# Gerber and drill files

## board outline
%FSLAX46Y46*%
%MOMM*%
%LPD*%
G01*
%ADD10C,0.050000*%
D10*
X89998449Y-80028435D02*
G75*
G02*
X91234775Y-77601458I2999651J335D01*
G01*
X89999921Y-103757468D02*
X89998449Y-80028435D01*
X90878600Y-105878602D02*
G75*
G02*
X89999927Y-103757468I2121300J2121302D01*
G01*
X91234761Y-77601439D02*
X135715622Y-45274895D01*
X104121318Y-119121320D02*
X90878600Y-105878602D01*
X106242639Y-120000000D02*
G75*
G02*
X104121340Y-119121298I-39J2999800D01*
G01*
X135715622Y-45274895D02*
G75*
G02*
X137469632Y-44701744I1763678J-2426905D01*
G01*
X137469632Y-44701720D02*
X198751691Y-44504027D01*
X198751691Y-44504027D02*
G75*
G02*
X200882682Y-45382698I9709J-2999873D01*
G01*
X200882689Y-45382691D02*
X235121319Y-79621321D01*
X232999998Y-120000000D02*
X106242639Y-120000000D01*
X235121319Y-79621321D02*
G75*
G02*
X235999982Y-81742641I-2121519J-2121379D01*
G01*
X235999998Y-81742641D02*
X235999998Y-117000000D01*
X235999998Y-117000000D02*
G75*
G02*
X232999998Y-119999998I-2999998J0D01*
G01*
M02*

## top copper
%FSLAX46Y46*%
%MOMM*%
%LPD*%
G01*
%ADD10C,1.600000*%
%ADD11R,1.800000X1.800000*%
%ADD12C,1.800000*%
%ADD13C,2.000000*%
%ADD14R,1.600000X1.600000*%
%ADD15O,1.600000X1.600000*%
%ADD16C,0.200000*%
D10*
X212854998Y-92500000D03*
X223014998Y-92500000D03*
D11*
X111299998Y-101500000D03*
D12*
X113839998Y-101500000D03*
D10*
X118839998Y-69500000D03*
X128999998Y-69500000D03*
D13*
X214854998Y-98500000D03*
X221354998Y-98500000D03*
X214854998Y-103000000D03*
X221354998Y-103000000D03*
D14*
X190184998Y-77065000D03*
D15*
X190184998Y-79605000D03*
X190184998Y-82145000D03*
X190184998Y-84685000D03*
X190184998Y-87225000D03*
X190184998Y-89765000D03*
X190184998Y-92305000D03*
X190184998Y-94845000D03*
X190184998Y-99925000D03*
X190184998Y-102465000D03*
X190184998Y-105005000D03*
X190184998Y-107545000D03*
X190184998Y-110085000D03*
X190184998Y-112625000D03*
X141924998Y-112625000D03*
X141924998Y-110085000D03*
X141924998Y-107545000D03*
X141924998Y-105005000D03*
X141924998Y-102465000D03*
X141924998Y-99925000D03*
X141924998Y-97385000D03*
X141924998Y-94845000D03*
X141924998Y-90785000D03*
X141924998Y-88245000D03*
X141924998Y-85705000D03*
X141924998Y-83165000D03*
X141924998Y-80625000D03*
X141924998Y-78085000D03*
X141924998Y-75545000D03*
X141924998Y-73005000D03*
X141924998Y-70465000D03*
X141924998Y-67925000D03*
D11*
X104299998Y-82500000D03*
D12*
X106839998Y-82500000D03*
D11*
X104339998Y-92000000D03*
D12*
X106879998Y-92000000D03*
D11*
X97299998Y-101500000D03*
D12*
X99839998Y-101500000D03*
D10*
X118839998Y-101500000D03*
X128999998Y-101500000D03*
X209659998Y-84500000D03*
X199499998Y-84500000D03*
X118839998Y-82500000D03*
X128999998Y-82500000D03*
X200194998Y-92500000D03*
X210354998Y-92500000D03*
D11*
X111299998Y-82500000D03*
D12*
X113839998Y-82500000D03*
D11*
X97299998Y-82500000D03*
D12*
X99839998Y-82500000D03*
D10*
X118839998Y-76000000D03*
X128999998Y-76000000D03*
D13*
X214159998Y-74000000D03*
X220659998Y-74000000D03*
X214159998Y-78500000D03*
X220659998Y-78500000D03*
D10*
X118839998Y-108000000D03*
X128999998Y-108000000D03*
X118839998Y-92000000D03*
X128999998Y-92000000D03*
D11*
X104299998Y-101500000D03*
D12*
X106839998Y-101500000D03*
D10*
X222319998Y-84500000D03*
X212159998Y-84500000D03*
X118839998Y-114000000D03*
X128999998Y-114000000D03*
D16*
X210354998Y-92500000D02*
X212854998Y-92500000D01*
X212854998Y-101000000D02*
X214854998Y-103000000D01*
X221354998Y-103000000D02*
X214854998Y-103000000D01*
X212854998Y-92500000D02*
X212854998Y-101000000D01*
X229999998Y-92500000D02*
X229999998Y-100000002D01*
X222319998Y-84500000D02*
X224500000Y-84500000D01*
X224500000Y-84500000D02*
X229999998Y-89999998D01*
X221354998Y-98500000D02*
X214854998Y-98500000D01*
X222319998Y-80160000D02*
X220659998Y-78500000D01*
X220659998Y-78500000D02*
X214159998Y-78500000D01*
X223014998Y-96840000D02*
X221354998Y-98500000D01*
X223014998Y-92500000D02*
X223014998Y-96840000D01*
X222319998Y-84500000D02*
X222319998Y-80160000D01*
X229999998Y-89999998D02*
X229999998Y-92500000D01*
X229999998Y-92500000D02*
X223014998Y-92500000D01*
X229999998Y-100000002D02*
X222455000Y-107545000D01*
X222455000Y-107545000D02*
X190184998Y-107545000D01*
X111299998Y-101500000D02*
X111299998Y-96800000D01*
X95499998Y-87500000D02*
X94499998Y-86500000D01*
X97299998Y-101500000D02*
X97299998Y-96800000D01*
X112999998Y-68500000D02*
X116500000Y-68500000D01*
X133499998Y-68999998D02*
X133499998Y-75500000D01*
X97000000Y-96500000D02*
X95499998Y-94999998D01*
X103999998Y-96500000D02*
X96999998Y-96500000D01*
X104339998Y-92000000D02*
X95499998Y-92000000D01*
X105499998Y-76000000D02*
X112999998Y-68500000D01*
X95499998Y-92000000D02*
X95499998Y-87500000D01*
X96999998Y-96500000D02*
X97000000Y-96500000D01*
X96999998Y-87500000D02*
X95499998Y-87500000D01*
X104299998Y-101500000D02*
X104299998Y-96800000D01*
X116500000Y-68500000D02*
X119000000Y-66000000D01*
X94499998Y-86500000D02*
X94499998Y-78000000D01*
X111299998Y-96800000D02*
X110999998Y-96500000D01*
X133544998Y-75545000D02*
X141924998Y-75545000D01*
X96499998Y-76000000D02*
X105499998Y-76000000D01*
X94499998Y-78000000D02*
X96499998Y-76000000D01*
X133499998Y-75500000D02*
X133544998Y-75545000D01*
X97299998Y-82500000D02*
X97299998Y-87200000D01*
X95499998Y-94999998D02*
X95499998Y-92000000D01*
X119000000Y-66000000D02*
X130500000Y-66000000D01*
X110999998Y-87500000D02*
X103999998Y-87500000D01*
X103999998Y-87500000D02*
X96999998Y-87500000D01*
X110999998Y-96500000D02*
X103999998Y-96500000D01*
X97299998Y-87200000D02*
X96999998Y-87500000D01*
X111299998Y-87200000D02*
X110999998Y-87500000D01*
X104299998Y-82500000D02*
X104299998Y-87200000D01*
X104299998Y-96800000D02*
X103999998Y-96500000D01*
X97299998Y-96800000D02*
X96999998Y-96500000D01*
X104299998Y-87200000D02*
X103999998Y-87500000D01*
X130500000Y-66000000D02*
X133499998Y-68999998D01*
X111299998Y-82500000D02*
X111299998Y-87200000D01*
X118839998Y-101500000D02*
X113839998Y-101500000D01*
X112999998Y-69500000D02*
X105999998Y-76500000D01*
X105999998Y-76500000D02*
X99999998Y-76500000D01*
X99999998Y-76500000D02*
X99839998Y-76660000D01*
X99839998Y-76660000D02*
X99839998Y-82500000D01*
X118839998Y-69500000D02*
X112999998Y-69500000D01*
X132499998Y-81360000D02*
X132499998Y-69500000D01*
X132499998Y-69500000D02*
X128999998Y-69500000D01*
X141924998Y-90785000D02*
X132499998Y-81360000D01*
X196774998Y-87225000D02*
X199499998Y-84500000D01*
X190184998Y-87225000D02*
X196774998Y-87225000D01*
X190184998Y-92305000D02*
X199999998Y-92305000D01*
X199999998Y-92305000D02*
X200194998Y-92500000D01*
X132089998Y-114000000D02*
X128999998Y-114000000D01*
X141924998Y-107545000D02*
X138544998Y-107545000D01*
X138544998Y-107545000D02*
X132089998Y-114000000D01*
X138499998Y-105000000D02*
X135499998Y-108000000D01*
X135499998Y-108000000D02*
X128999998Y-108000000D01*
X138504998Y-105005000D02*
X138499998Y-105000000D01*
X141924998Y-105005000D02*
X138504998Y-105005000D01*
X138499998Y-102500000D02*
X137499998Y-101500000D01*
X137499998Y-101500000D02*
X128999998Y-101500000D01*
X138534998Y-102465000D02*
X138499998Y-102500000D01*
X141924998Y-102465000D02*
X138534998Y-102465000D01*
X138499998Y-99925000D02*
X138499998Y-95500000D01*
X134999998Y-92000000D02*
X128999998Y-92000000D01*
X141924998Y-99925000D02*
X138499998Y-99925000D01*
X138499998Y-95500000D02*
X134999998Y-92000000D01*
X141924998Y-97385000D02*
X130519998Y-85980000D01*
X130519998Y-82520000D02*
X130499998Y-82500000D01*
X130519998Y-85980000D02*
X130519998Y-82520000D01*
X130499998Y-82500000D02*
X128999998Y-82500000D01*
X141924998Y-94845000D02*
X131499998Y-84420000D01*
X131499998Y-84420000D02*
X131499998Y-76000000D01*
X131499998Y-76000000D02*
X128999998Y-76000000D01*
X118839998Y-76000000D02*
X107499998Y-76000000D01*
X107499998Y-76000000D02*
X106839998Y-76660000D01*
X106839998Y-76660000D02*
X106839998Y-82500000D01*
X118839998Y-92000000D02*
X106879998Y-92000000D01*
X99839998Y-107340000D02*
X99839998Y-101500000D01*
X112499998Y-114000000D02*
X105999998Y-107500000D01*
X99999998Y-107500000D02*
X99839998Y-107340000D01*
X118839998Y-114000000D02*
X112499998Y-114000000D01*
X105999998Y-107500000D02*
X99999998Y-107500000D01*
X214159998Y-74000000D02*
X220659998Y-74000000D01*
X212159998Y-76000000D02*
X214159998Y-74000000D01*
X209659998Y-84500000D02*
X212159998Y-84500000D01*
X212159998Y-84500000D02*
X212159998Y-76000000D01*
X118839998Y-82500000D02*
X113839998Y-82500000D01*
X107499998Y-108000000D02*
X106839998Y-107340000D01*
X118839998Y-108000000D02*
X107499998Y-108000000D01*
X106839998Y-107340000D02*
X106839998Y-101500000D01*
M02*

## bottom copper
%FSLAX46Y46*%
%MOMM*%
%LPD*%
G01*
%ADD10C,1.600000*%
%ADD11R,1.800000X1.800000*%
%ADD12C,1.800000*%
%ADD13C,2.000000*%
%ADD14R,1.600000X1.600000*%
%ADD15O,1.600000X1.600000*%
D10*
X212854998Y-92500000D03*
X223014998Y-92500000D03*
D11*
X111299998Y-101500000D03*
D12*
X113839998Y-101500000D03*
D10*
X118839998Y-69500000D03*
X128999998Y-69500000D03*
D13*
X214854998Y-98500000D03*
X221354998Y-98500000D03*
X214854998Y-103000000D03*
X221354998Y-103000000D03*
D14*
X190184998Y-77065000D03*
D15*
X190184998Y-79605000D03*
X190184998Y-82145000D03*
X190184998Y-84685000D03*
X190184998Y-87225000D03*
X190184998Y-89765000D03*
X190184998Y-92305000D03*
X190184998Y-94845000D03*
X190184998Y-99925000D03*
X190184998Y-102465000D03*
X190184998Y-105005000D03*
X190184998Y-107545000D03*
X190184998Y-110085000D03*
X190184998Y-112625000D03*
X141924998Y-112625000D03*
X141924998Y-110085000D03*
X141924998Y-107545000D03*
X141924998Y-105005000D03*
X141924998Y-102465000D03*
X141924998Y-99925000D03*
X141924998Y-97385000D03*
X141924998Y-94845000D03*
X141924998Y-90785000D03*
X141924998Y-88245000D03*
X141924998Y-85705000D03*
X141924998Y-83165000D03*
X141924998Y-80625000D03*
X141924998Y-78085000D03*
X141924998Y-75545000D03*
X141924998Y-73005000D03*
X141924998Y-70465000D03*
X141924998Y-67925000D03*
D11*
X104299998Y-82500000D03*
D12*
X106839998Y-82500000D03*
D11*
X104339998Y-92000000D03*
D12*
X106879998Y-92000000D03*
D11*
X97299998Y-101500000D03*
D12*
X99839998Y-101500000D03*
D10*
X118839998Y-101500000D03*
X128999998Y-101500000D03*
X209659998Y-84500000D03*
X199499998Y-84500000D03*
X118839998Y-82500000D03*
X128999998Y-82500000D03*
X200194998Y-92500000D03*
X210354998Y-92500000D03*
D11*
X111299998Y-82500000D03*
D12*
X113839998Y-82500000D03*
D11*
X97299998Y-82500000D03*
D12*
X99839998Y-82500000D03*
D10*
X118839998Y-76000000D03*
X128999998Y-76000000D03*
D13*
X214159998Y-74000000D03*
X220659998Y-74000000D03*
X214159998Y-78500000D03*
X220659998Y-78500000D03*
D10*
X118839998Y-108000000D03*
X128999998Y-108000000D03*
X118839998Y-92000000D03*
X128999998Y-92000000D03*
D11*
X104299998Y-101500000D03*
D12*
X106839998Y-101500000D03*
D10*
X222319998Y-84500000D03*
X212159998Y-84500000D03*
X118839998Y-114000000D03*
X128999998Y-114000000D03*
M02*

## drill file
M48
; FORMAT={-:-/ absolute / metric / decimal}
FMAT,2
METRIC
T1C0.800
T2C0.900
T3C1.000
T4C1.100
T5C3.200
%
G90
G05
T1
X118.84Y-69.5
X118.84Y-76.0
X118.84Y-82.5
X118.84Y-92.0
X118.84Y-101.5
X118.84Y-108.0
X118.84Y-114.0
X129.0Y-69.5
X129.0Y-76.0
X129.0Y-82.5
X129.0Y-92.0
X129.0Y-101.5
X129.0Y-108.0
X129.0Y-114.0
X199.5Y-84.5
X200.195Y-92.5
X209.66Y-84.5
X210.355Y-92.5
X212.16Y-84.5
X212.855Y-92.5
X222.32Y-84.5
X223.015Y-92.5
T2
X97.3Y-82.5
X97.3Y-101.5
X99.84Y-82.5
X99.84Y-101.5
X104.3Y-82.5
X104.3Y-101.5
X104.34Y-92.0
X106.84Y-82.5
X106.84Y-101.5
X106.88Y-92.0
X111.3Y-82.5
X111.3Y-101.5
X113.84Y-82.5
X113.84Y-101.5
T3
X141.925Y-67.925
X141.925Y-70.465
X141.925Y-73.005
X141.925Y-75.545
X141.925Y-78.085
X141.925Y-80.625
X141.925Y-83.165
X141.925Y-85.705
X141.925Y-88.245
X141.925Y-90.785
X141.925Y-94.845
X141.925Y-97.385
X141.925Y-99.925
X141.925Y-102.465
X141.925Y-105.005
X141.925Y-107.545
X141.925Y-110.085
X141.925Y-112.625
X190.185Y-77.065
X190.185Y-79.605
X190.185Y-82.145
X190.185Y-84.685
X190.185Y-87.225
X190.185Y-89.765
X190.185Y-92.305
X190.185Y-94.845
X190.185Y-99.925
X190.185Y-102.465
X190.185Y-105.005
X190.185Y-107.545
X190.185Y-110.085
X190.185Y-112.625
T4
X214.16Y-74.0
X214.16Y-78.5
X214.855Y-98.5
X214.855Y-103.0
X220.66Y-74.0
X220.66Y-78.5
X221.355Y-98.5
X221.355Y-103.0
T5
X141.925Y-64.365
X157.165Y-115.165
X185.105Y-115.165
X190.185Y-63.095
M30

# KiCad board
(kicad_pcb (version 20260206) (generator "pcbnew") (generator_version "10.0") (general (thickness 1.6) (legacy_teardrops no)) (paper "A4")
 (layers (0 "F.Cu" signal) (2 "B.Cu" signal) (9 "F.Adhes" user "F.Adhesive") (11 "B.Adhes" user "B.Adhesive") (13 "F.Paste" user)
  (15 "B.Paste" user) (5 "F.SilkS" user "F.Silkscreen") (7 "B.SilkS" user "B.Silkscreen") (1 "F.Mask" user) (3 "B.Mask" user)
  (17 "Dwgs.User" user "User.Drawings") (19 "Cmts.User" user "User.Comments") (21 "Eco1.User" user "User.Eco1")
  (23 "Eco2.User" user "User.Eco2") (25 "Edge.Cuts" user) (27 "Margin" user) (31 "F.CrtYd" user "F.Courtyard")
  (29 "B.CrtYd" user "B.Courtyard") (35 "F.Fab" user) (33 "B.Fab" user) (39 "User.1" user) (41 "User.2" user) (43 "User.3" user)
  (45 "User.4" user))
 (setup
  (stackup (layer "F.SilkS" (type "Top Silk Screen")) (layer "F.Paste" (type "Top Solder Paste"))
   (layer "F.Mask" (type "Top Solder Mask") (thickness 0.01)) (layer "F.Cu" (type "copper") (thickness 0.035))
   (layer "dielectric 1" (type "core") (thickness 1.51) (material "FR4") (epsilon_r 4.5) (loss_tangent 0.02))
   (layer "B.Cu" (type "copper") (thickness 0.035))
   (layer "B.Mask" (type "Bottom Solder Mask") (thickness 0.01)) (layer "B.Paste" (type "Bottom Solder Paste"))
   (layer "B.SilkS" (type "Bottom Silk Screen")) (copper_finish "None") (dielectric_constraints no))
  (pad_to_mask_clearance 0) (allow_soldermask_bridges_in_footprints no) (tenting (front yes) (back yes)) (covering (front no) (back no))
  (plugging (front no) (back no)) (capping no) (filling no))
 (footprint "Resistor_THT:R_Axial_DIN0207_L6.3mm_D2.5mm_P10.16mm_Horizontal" (layer "F.Cu") (at 212.854998 92.5)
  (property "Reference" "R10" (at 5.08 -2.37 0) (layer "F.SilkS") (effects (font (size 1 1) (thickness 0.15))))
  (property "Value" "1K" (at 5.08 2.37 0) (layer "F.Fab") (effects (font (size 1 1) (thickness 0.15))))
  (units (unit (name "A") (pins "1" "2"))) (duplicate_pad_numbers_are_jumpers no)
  (pad "1" thru_hole circle (at 0 0) (size 1.6 1.6) (drill 0.8) (layers "*.Cu" "*.Mask") (remove_unused_layers no) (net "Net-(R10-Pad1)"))
  (pad "2" thru_hole circle (at 10.16 0) (size 1.6 1.6) (drill 0.8) (layers "*.Cu" "*.Mask") (remove_unused_layers no) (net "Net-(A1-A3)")))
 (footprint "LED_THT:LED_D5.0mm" (layer "F.Cu") (at 111.299998 101.5)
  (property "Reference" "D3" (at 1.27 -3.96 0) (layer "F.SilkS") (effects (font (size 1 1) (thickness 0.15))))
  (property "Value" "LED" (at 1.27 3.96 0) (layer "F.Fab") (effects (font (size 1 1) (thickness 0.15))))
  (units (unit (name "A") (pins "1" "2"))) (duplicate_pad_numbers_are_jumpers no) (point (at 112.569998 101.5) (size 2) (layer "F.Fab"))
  (pad "1" thru_hole rect (at 0 0) (size 1.8 1.8) (drill 0.9) (layers "*.Cu" "*.Mask") (remove_unused_layers no) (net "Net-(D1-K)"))
  (pad "2" thru_hole circle (at 2.54 0) (size 1.8 1.8) (drill 0.9) (layers "*.Cu" "*.Mask") (remove_unused_layers no) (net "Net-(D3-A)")))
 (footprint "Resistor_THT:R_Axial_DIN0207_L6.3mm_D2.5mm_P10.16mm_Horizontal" (layer "F.Cu") (at 118.839998 69.5)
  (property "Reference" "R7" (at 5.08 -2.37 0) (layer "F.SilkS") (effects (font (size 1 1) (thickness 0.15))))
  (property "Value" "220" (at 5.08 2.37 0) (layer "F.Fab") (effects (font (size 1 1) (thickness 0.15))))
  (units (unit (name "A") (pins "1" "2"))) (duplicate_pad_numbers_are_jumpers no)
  (pad "1" thru_hole circle (at 0 0) (size 1.6 1.6) (drill 0.8) (layers "*.Cu" "*.Mask") (remove_unused_layers no) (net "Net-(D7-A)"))
  (pad "2" thru_hole circle (at 10.16 0) (size 1.6 1.6) (drill 0.8) (layers "*.Cu" "*.Mask") (remove_unused_layers no) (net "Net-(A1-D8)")))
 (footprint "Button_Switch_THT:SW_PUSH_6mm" (layer "F.Cu") (at 214.854998 98.5)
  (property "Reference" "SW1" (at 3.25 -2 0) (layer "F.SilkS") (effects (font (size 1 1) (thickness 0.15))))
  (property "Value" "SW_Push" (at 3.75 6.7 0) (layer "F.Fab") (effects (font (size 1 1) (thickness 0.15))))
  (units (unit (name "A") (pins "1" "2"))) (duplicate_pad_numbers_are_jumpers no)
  (pad "1" thru_hole circle (at 0 0 90) (size 2 2) (drill 1.1) (layers "*.Cu" "*.Mask") (remove_unused_layers no) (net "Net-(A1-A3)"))
  (pad "1" thru_hole circle (at 6.5 0 90) (size 2 2) (drill 1.1) (layers "*.Cu" "*.Mask") (remove_unused_layers no) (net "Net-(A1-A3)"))
  (pad "2" thru_hole circle (at 0 4.5 90) (size 2 2) (drill 1.1) (layers "*.Cu" "*.Mask") (remove_unused_layers no) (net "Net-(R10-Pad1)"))
  (pad "2" thru_hole circle (at 6.5 4.5 90) (size 2 2) (drill 1.1) (layers "*.Cu" "*.Mask") (remove_unused_layers no) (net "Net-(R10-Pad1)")))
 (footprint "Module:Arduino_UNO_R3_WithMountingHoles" (layer "F.Cu") (at 190.184998 77.065 -90)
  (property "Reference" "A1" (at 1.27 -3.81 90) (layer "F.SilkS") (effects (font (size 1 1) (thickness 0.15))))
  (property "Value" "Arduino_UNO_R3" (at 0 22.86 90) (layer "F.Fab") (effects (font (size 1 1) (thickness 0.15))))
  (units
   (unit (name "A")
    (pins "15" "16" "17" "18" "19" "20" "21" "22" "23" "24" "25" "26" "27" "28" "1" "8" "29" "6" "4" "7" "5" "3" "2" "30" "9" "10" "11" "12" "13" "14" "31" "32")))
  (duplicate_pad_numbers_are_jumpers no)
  (pad "" np_thru_hole circle (at -13.97 0) (size 3.2 3.2) (drill 3.2) (layers "*.Cu" "*.Mask"))
  (pad "" np_thru_hole circle (at -12.7 48.26) (size 3.2 3.2) (drill 3.2) (layers "*.Cu" "*.Mask"))
  (pad "" np_thru_hole circle (at 38.1 5.08) (size 3.2 3.2) (drill 3.2) (layers "*.Cu" "*.Mask"))
  (pad "" np_thru_hole circle (at 38.1 33.02) (size 3.2 3.2) (drill 3.2) (layers "*.Cu" "*.Mask"))
  (pad "1" thru_hole rect (at 0 0) (size 1.6 1.6) (drill 1) (layers "*.Cu" "*.Mask") (remove_unused_layers no)
   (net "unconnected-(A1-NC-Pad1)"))
  (pad "2" thru_hole oval (at 2.54 0) (size 1.6 1.6) (drill 1) (layers "*.Cu" "*.Mask") (remove_unused_layers no)
   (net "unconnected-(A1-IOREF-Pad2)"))
  (pad "3" thru_hole oval (at 5.08 0) (size 1.6 1.6) (drill 1) (layers "*.Cu" "*.Mask") (remove_unused_layers no)
   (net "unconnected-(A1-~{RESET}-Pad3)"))
  (pad "4" thru_hole oval (at 7.62 0) (size 1.6 1.6) (drill 1) (layers "*.Cu" "*.Mask") (remove_unused_layers no)
   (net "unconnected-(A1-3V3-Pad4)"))
  (pad "5" thru_hole oval (at 10.16 0) (size 1.6 1.6) (drill 1) (layers "*.Cu" "*.Mask") (remove_unused_layers no) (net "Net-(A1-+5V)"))
  (pad "6" thru_hole oval (at 12.7 0) (size 1.6 1.6) (drill 1) (layers "*.Cu" "*.Mask") (remove_unused_layers no)
   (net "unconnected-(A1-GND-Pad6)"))
  (pad "7" thru_hole oval (at 15.24 0) (size 1.6 1.6) (drill 1) (layers "*.Cu" "*.Mask") (remove_unused_layers no) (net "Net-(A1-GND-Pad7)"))
  (pad "8" thru_hole oval (at 17.78 0) (size 1.6 1.6) (drill 1) (layers "*.Cu" "*.Mask") (remove_unused_layers no)
   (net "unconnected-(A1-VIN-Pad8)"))
  (pad "9" thru_hole oval (at 22.86 0) (size 1.6 1.6) (drill 1) (layers "*.Cu" "*.Mask") (remove_unused_layers no)
   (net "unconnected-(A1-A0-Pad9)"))
  (pad "10" thru_hole oval (at 25.4 0) (size 1.6 1.6) (drill 1) (layers "*.Cu" "*.Mask") (remove_unused_layers no)
   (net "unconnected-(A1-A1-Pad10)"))
  (pad "11" thru_hole oval (at 27.94 0) (size 1.6 1.6) (drill 1) (layers "*.Cu" "*.Mask") (remove_unused_layers no)
   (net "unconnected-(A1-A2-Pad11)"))
  (pad "12" thru_hole oval (at 30.48 0) (size 1.6 1.6) (drill 1) (layers "*.Cu" "*.Mask") (remove_unused_layers no) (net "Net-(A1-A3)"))
  (pad "13" thru_hole oval (at 33.02 0) (size 1.6 1.6) (drill 1) (layers "*.Cu" "*.Mask") (remove_unused_layers no)
   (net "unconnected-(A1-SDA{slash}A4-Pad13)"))
  (pad "14" thru_hole oval (at 35.56 0) (size 1.6 1.6) (drill 1) (layers "*.Cu" "*.Mask") (remove_unused_layers no)
   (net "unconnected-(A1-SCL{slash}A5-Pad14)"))
  (pad "15" thru_hole oval (at 35.56 48.26) (size 1.6 1.6) (drill 1) (layers "*.Cu" "*.Mask") (remove_unused_layers no)
   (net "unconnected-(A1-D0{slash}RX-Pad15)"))
  (pad "16" thru_hole oval (at 33.02 48.26) (size 1.6 1.6) (drill 1) (layers "*.Cu" "*.Mask") (remove_unused_layers no)
   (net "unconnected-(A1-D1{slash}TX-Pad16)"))
  (pad "17" thru_hole oval (at 30.48 48.26) (size 1.6 1.6) (drill 1) (layers "*.Cu" "*.Mask") (remove_unused_layers no) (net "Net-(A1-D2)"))
  (pad "18" thru_hole oval (at 27.94 48.26) (size 1.6 1.6) (drill 1) (layers "*.Cu" "*.Mask") (remove_unused_layers no) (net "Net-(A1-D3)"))
  (pad "19" thru_hole oval (at 25.4 48.26) (size 1.6 1.6) (drill 1) (layers "*.Cu" "*.Mask") (remove_unused_layers no) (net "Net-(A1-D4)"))
  (pad "20" thru_hole oval (at 22.86 48.26) (size 1.6 1.6) (drill 1) (layers "*.Cu" "*.Mask") (remove_unused_layers no) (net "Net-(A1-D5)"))
  (pad "21" thru_hole oval (at 20.32 48.26) (size 1.6 1.6) (drill 1) (layers "*.Cu" "*.Mask") (remove_unused_layers no) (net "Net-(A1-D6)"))
  (pad "22" thru_hole oval (at 17.78 48.26) (size 1.6 1.6) (drill 1) (layers "*.Cu" "*.Mask") (remove_unused_layers no) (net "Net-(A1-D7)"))
  (pad "23" thru_hole oval (at 13.72 48.26) (size 1.6 1.6) (drill 1) (layers "*.Cu" "*.Mask") (remove_unused_layers no) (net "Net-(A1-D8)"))
  (pad "24" thru_hole oval (at 11.18 48.26) (size 1.6 1.6) (drill 1) (layers "*.Cu" "*.Mask") (remove_unused_layers no)
   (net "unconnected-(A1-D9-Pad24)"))
  (pad "25" thru_hole oval (at 8.64 48.26) (size 1.6 1.6) (drill 1) (layers "*.Cu" "*.Mask") (remove_unused_layers no)
   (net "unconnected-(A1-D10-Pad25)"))
  (pad "26" thru_hole oval (at 6.1 48.26) (size 1.6 1.6) (drill 1) (layers "*.Cu" "*.Mask") (remove_unused_layers no)
   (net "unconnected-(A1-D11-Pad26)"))
  (pad "27" thru_hole oval (at 3.56 48.26) (size 1.6 1.6) (drill 1) (layers "*.Cu" "*.Mask") (remove_unused_layers no)
   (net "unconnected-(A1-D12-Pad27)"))
  (pad "28" thru_hole oval (at 1.02 48.26) (size 1.6 1.6) (drill 1) (layers "*.Cu" "*.Mask") (remove_unused_layers no)
   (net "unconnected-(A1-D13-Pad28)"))
  (pad "29" thru_hole oval (at -1.52 48.26) (size 1.6 1.6) (drill 1) (layers "*.Cu" "*.Mask") (remove_unused_layers no) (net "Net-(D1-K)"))
  (pad "30" thru_hole oval (at -4.06 48.26) (size 1.6 1.6) (drill 1) (layers "*.Cu" "*.Mask") (remove_unused_layers no)
   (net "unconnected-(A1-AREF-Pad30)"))
  (pad "31" thru_hole oval (at -6.6 48.26) (size 1.6 1.6) (drill 1) (layers "*.Cu" "*.Mask") (remove_unused_layers no)
   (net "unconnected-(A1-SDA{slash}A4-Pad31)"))
  (pad "32" thru_hole oval (at -9.14 48.26) (size 1.6 1.6) (drill 1) (layers "*.Cu" "*.Mask") (remove_unused_layers no)
   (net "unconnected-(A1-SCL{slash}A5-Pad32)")))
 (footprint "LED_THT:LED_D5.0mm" (layer "F.Cu") (at 104.299998 82.5)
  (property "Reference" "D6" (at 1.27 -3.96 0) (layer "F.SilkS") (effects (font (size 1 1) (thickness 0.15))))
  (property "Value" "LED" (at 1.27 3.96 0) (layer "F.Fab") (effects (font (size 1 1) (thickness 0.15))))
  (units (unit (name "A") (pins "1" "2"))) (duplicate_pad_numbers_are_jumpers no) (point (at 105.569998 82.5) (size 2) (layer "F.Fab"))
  (pad "1" thru_hole rect (at 0 0) (size 1.8 1.8) (drill 0.9) (layers "*.Cu" "*.Mask") (remove_unused_layers no) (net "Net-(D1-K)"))
  (pad "2" thru_hole circle (at 2.54 0) (size 1.8 1.8) (drill 0.9) (layers "*.Cu" "*.Mask") (remove_unused_layers no) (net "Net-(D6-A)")))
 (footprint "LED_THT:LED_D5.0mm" (layer "F.Cu") (at 104.339998 92)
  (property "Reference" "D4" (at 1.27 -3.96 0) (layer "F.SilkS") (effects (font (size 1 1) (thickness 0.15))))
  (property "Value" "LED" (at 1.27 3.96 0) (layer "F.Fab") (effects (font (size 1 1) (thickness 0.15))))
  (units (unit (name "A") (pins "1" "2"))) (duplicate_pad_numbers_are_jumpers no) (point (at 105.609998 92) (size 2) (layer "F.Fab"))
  (pad "1" thru_hole rect (at 0 0) (size 1.8 1.8) (drill 0.9) (layers "*.Cu" "*.Mask") (remove_unused_layers no) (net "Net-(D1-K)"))
  (pad "2" thru_hole circle (at 2.54 0) (size 1.8 1.8) (drill 0.9) (layers "*.Cu" "*.Mask") (remove_unused_layers no) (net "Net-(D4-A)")))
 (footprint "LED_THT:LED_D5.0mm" (layer "F.Cu") (at 97.299998 101.5)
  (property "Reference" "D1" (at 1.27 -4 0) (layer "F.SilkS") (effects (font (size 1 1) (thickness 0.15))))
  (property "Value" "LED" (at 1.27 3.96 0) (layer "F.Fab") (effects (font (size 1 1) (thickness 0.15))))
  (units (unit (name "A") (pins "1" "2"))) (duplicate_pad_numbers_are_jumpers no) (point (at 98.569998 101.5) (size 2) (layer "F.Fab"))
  (pad "1" thru_hole rect (at 0 0) (size 1.8 1.8) (drill 0.9) (layers "*.Cu" "*.Mask") (remove_unused_layers no) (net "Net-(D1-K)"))
  (pad "2" thru_hole circle (at 2.54 0) (size 1.8 1.8) (drill 0.9) (layers "*.Cu" "*.Mask") (remove_unused_layers no) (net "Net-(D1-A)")))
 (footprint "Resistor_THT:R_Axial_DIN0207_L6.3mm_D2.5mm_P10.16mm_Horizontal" (layer "F.Cu") (at 118.839998 101.5)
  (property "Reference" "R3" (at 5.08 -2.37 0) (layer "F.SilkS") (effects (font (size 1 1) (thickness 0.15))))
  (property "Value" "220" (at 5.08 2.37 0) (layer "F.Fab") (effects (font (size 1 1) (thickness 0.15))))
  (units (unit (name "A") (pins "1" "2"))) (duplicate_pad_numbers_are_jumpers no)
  (pad "1" thru_hole circle (at 0 0) (size 1.6 1.6) (drill 0.8) (layers "*.Cu" "*.Mask") (remove_unused_layers no) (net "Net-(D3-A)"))
  (pad "2" thru_hole circle (at 10.16 0) (size 1.6 1.6) (drill 0.8) (layers "*.Cu" "*.Mask") (remove_unused_layers no) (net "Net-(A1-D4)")))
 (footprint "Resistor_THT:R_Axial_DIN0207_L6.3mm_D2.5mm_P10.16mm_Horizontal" (layer "F.Cu") (at 209.659998 84.5 180)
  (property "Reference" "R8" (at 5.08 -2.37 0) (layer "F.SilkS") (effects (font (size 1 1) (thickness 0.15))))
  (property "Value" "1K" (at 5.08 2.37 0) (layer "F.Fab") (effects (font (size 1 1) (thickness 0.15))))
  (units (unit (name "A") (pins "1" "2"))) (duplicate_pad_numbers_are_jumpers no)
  (pad "1" thru_hole circle (at 0 0 180) (size 1.6 1.6) (drill 0.8) (layers "*.Cu" "*.Mask") (remove_unused_layers no) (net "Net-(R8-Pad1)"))
  (pad "2" thru_hole circle (at 10.16 0 180) (size 1.6 1.6) (drill 0.8) (layers "*.Cu" "*.Mask") (remove_unused_layers no)
   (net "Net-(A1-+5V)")))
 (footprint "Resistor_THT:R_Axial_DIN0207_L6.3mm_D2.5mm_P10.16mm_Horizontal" (layer "F.Cu") (at 118.839998 82.5)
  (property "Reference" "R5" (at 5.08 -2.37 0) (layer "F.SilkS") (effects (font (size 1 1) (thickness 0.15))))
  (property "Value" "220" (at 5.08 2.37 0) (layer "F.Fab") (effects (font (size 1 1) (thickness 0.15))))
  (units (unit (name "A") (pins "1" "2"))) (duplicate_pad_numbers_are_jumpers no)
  (pad "1" thru_hole circle (at 0 0) (size 1.6 1.6) (drill 0.8) (layers "*.Cu" "*.Mask") (remove_unused_layers no) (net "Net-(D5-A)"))
  (pad "2" thru_hole circle (at 10.16 0) (size 1.6 1.6) (drill 0.8) (layers "*.Cu" "*.Mask") (remove_unused_layers no) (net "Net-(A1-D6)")))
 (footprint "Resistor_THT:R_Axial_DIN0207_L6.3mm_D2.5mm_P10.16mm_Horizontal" (layer "F.Cu") (at 200.194998 92.5)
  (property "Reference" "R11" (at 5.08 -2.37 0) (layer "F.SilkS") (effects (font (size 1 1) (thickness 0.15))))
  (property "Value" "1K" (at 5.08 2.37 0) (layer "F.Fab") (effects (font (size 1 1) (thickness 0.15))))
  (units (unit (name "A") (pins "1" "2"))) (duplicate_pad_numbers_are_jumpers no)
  (pad "1" thru_hole circle (at 0 0) (size 1.6 1.6) (drill 0.8) (layers "*.Cu" "*.Mask") (remove_unused_layers no) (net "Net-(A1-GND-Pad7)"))
  (pad "2" thru_hole circle (at 10.16 0) (size 1.6 1.6) (drill 0.8) (layers "*.Cu" "*.Mask") (remove_unused_layers no)
   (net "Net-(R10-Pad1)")))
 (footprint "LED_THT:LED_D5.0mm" (layer "F.Cu") (at 111.299998 82.5)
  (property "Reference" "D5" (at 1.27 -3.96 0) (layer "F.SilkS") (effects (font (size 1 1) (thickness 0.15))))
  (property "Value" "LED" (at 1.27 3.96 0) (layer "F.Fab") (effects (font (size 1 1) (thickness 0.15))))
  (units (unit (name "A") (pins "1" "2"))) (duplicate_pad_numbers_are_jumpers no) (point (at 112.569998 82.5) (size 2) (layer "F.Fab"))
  (pad "1" thru_hole rect (at 0 0) (size 1.8 1.8) (drill 0.9) (layers "*.Cu" "*.Mask") (remove_unused_layers no) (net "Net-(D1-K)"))
  (pad "2" thru_hole circle (at 2.54 0) (size 1.8 1.8) (drill 0.9) (layers "*.Cu" "*.Mask") (remove_unused_layers no) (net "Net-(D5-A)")))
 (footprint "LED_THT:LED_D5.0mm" (layer "F.Cu") (at 97.299998 82.5)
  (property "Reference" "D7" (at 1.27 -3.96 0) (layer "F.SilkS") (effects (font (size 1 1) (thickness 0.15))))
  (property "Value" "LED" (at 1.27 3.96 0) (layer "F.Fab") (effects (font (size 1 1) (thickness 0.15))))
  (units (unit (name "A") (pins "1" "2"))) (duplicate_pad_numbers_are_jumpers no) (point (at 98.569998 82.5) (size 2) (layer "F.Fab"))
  (pad "1" thru_hole rect (at 0 0) (size 1.8 1.8) (drill 0.9) (layers "*.Cu" "*.Mask") (remove_unused_layers no) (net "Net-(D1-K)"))
  (pad "2" thru_hole circle (at 2.54 0) (size 1.8 1.8) (drill 0.9) (layers "*.Cu" "*.Mask") (remove_unused_layers no) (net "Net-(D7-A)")))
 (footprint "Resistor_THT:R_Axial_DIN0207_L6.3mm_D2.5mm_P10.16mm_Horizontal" (layer "F.Cu") (at 118.839998 76)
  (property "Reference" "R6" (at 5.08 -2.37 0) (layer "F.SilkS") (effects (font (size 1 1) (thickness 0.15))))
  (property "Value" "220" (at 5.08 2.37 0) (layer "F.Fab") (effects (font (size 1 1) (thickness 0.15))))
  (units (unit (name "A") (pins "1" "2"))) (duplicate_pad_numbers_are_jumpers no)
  (pad "1" thru_hole circle (at 0 0) (size 1.6 1.6) (drill 0.8) (layers "*.Cu" "*.Mask") (remove_unused_layers no) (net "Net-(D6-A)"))
  (pad "2" thru_hole circle (at 10.16 0) (size 1.6 1.6) (drill 0.8) (layers "*.Cu" "*.Mask") (remove_unused_layers no) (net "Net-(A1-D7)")))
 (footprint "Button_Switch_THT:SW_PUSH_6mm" (layer "F.Cu") (at 214.159998 74)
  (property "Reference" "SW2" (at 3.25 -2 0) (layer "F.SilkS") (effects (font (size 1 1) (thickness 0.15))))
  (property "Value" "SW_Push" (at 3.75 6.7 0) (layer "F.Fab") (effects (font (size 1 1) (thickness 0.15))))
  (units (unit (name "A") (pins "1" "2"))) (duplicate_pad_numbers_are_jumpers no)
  (pad "1" thru_hole circle (at 0 0 90) (size 2 2) (drill 1.1) (layers "*.Cu" "*.Mask") (remove_unused_layers no) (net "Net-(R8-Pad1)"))
  (pad "1" thru_hole circle (at 6.5 0 90) (size 2 2) (drill 1.1) (layers "*.Cu" "*.Mask") (remove_unused_layers no) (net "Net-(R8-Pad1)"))
  (pad "2" thru_hole circle (at 0 4.5 90) (size 2 2) (drill 1.1) (layers "*.Cu" "*.Mask") (remove_unused_layers no) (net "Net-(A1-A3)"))
  (pad "2" thru_hole circle (at 6.5 4.5 90) (size 2 2) (drill 1.1) (layers "*.Cu" "*.Mask") (remove_unused_layers no) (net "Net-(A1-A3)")))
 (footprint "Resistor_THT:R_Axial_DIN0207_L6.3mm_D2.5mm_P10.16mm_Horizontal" (layer "F.Cu") (at 118.839998 108)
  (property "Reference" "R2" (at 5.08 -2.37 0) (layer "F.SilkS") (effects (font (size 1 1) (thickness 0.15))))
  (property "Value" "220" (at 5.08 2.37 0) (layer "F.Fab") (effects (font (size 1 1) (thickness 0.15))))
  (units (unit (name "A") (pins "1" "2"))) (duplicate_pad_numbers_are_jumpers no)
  (pad "1" thru_hole circle (at 0 0) (size 1.6 1.6) (drill 0.8) (layers "*.Cu" "*.Mask") (remove_unused_layers no) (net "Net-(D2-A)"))
  (pad "2" thru_hole circle (at 10.16 0) (size 1.6 1.6) (drill 0.8) (layers "*.Cu" "*.Mask") (remove_unused_layers no) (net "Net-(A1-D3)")))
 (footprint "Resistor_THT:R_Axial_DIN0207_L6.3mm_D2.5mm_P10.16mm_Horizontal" (layer "F.Cu") (at 118.839998 92)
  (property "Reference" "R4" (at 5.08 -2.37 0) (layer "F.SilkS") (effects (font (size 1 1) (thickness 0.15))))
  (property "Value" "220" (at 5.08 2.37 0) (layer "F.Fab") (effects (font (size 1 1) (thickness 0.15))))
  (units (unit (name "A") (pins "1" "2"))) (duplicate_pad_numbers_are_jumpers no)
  (pad "1" thru_hole circle (at 0 0) (size 1.6 1.6) (drill 0.8) (layers "*.Cu" "*.Mask") (remove_unused_layers no) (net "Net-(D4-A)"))
  (pad "2" thru_hole circle (at 10.16 0) (size 1.6 1.6) (drill 0.8) (layers "*.Cu" "*.Mask") (remove_unused_layers no) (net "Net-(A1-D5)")))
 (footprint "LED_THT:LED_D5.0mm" (layer "F.Cu") (at 104.299998 101.5)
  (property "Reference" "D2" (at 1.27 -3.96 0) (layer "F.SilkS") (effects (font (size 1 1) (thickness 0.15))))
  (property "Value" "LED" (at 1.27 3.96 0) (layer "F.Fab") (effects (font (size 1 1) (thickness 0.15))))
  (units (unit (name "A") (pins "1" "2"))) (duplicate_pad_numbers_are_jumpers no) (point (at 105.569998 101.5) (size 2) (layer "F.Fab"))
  (pad "1" thru_hole rect (at 0 0) (size 1.8 1.8) (drill 0.9) (layers "*.Cu" "*.Mask") (remove_unused_layers no) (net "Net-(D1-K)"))
  (pad "2" thru_hole circle (at 2.54 0) (size 1.8 1.8) (drill 0.9) (layers "*.Cu" "*.Mask") (remove_unused_layers no) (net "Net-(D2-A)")))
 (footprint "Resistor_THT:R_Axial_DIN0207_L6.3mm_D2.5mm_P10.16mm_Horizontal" (layer "F.Cu") (at 222.319998 84.5 180)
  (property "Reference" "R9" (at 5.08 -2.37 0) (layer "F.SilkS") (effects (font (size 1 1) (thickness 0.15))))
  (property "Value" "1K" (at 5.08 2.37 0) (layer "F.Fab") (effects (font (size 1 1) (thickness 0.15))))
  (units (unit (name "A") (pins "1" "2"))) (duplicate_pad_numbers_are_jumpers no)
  (pad "1" thru_hole circle (at 0 0 180) (size 1.6 1.6) (drill 0.8) (layers "*.Cu" "*.Mask") (remove_unused_layers no) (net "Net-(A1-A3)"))
  (pad "2" thru_hole circle (at 10.16 0 180) (size 1.6 1.6) (drill 0.8) (layers "*.Cu" "*.Mask") (remove_unused_layers no)
   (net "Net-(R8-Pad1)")))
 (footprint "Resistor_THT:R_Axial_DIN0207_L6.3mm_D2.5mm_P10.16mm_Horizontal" (layer "F.Cu") (at 118.839998 114)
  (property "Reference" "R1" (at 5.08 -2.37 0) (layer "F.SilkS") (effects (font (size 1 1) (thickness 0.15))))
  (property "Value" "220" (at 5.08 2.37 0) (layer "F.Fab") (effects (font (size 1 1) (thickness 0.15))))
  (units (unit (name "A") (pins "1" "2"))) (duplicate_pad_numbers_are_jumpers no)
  (pad "1" thru_hole circle (at 0 0) (size 1.6 1.6) (drill 0.8) (layers "*.Cu" "*.Mask") (remove_unused_layers no) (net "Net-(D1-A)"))
  (pad "2" thru_hole circle (at 10.16 0) (size 1.6 1.6) (drill 0.8) (layers "*.Cu" "*.Mask") (remove_unused_layers no) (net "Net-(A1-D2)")))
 (gr_arc (start 89.998449 80.028435) (mid 90.325259 78.666523) (end 91.234761 77.601439) (stroke (width 0.05) (type default))
  (layer "Edge.Cuts"))
 (gr_line (start 89.999921 103.757468) (end 89.998449 80.028435) (stroke (width 0.05) (type default)) (layer "Edge.Cuts"))
 (gr_arc (start 90.8786 105.878602) (mid 90.228319 104.905418) (end 89.999921 103.757468) (stroke (width 0.05) (type default))
  (layer "Edge.Cuts"))
 (gr_line (start 91.234761 77.601439) (end 135.715622 45.274895) (stroke (width 0.05) (type default)) (layer "Edge.Cuts"))
 (gr_line (start 104.121318 119.12132) (end 90.8786 105.878602) (stroke (width 0.05) (type default)) (layer "Edge.Cuts"))
 (gr_arc (start 106.242639 120) (mid 105.09458 119.771652) (end 104.121318 119.12132) (stroke (width 0.05) (type default))
  (layer "Edge.Cuts"))
 (gr_arc (start 135.715622 45.274895) (mid 136.547463 44.850101) (end 137.469632 44.70172) (stroke (width 0.05) (type default))
  (layer "Edge.Cuts"))
 (gr_line (start 137.469632 44.70172) (end 198.751691 44.504027) (stroke (width 0.05) (type default)) (layer "Edge.Cuts"))
 (gr_arc (start 198.751691 44.504027) (mid 199.904953 44.730516) (end 200.882689 45.382691) (stroke (width 0.05) (type default))
  (layer "Edge.Cuts"))
 (gr_line (start 200.882689 45.382691) (end 235.121319 79.621321) (stroke (width 0.05) (type default)) (layer "Edge.Cuts"))
 (gr_line (start 232.999998 120) (end 106.242639 120) (stroke (width 0.05) (type default)) (layer "Edge.Cuts"))
 (gr_arc (start 235.121319 79.621321) (mid 235.771624 80.594593) (end 235.999998 81.742641) (stroke (width 0.05) (type default))
  (layer "Edge.Cuts"))
 (gr_line (start 235.999998 81.742641) (end 235.999998 117) (stroke (width 0.05) (type default)) (layer "Edge.Cuts"))
 (gr_arc (start 235.999998 117) (mid 235.121318 119.12132) (end 232.999998 120) (stroke (width 0.05) (type default)) (layer "Edge.Cuts"))
 (segment (start 210.354998 92.5) (end 212.854998 92.5) (width 0.2) (layer "F.Cu") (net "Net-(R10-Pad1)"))
 (segment (start 212.854998 101) (end 214.854998 103) (width 0.2) (layer "F.Cu") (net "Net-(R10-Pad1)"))
 (segment (start 221.354998 103) (end 214.854998 103) (width 0.2) (layer "F.Cu") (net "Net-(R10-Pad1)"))
 (segment (start 212.854998 92.5) (end 212.854998 101) (width 0.2) (layer "F.Cu") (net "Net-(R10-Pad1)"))
 (segment (start 229.999998 92.5) (end 229.999998 100.000002) (width 0.2) (layer "F.Cu") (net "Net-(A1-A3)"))
 (segment (start 222.319998 84.5) (end 224.5 84.5) (width 0.2) (layer "F.Cu") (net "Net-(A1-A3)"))
 (segment (start 224.5 84.5) (end 229.999998 89.999998) (width 0.2) (layer "F.Cu") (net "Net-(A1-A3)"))
 (segment (start 221.354998 98.5) (end 214.854998 98.5) (width 0.2) (layer "F.Cu") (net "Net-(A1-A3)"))
 (segment (start 222.319998 80.16) (end 220.659998 78.5) (width 0.2) (layer "F.Cu") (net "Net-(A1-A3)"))
 (segment (start 220.659998 78.5) (end 214.159998 78.5) (width 0.2) (layer "F.Cu") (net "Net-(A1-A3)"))
 (segment (start 223.014998 96.84) (end 221.354998 98.5) (width 0.2) (layer "F.Cu") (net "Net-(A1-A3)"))
 (segment (start 223.014998 92.5) (end 223.014998 96.84) (width 0.2) (layer "F.Cu") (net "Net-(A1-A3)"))
 (segment (start 222.319998 84.5) (end 222.319998 80.16) (width 0.2) (layer "F.Cu") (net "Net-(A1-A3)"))
 (segment (start 229.999998 89.999998) (end 229.999998 92.5) (width 0.2) (layer "F.Cu") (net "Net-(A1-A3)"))
 (segment (start 229.999998 92.5) (end 223.014998 92.5) (width 0.2) (layer "F.Cu") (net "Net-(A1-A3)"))
 (segment (start 229.999998 100.000002) (end 222.455 107.545) (width 0.2) (layer "F.Cu") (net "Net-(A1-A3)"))
 (segment (start 222.455 107.545) (end 190.184998 107.545) (width 0.2) (layer "F.Cu") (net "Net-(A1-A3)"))
 (segment (start 111.299998 101.5) (end 111.299998 96.8) (width 0.2) (layer "F.Cu") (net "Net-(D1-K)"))
 (segment (start 95.499998 87.5) (end 94.499998 86.5) (width 0.2) (layer "F.Cu") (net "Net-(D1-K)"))
 (segment (start 97.299998 101.5) (end 97.299998 96.8) (width 0.2) (layer "F.Cu") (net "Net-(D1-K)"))
 (segment (start 112.999998 68.5) (end 116.5 68.5) (width 0.2) (layer "F.Cu") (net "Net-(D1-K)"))
 (segment (start 133.499998 68.999998) (end 133.499998 75.5) (width 0.2) (layer "F.Cu") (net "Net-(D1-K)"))
 (segment (start 97 96.5) (end 95.499998 94.999998) (width 0.2) (layer "F.Cu") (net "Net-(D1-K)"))
 (segment (start 103.999998 96.5) (end 96.999998 96.5) (width 0.2) (layer "F.Cu") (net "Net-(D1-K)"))
 (segment (start 104.339998 92) (end 95.499998 92) (width 0.2) (layer "F.Cu") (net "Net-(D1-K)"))
 (segment (start 105.499998 76) (end 112.999998 68.5) (width 0.2) (layer "F.Cu") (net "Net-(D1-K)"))
 (segment (start 95.499998 92) (end 95.499998 87.5) (width 0.2) (layer "F.Cu") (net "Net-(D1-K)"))
 (segment (start 96.999998 96.5) (end 97 96.5) (width 0.2) (layer "F.Cu") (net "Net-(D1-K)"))
 (segment (start 96.999998 87.5) (end 95.499998 87.5) (width 0.2) (layer "F.Cu") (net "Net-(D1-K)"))
 (segment (start 104.299998 101.5) (end 104.299998 96.8) (width 0.2) (layer "F.Cu") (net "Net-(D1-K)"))
 (segment (start 116.5 68.5) (end 119 66) (width 0.2) (layer "F.Cu") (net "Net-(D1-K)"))
 (segment (start 94.499998 86.5) (end 94.499998 78) (width 0.2) (layer "F.Cu") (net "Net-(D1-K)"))
 (segment (start 111.299998 96.8) (end 110.999998 96.5) (width 0.2) (layer "F.Cu") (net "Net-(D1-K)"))
 (segment (start 133.544998 75.545) (end 141.924998 75.545) (width 0.2) (layer "F.Cu") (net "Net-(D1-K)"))
 (segment (start 96.499998 76) (end 105.499998 76) (width 0.2) (layer "F.Cu") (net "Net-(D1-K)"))
 (segment (start 94.499998 78) (end 96.499998 76) (width 0.2) (layer "F.Cu") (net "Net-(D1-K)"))
 (segment (start 133.499998 75.5) (end 133.544998 75.545) (width 0.2) (layer "F.Cu") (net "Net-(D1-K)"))
 (segment (start 97.299998 82.5) (end 97.299998 87.2) (width 0.2) (layer "F.Cu") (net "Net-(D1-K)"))
 (segment (start 95.499998 94.999998) (end 95.499998 92) (width 0.2) (layer "F.Cu") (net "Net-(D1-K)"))
 (segment (start 119 66) (end 130.5 66) (width 0.2) (layer "F.Cu") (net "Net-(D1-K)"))
 (segment (start 110.999998 87.5) (end 103.999998 87.5) (width 0.2) (layer "F.Cu") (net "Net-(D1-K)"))
 (segment (start 103.999998 87.5) (end 96.999998 87.5) (width 0.2) (layer "F.Cu") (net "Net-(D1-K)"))
 (segment (start 110.999998 96.5) (end 103.999998 96.5) (width 0.2) (layer "F.Cu") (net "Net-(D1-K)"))
 (segment (start 97.299998 87.2) (end 96.999998 87.5) (width 0.2) (layer "F.Cu") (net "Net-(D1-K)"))
 (segment (start 111.299998 87.2) (end 110.999998 87.5) (width 0.2) (layer "F.Cu") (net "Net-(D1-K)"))
 (segment (start 104.299998 82.5) (end 104.299998 87.2) (width 0.2) (layer "F.Cu") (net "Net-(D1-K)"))
 (segment (start 104.299998 96.8) (end 103.999998 96.5) (width 0.2) (layer "F.Cu") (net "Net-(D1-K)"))
 (segment (start 97.299998 96.8) (end 96.999998 96.5) (width 0.2) (layer "F.Cu") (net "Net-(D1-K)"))
 (segment (start 104.299998 87.2) (end 103.999998 87.5) (width 0.2) (layer "F.Cu") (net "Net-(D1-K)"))
 (segment (start 130.5 66) (end 133.499998 68.999998) (width 0.2) (layer "F.Cu") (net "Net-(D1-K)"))
 (segment (start 111.299998 82.5) (end 111.299998 87.2) (width 0.2) (layer "F.Cu") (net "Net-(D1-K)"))
 (segment (start 118.839998 101.5) (end 113.839998 101.5) (width 0.2) (layer "F.Cu") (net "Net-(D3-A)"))
 (segment (start 112.999998 69.5) (end 105.999998 76.5) (width 0.2) (layer "F.Cu") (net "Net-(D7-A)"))
 (segment (start 105.999998 76.5) (end 99.999998 76.5) (width 0.2) (layer "F.Cu") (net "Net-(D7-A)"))
 (segment (start 99.999998 76.5) (end 99.839998 76.66) (width 0.2) (layer "F.Cu") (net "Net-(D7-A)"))
 (segment (start 99.839998 76.66) (end 99.839998 82.5) (width 0.2) (layer "F.Cu") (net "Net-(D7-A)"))
 (segment (start 118.839998 69.5) (end 112.999998 69.5) (width 0.2) (layer "F.Cu") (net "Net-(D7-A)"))
 (segment (start 132.499998 81.36) (end 132.499998 69.5) (width 0.2) (layer "F.Cu") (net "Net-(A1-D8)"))
 (segment (start 132.499998 69.5) (end 128.999998 69.5) (width 0.2) (layer "F.Cu") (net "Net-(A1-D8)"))
 (segment (start 141.924998 90.785) (end 132.499998 81.36) (width 0.2) (layer "F.Cu") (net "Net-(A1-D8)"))
 (segment (start 196.774998 87.225) (end 199.499998 84.5) (width 0.2) (layer "F.Cu") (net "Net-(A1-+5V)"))
 (segment (start 190.184998 87.225) (end 196.774998 87.225) (width 0.2) (layer "F.Cu") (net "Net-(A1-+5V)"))
 (segment (start 190.184998 92.305) (end 199.999998 92.305) (width 0.2) (layer "F.Cu") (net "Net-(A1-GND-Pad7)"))
 (segment (start 199.999998 92.305) (end 200.194998 92.5) (width 0.2) (layer "F.Cu") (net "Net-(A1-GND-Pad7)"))
 (segment (start 132.089998 114) (end 128.999998 114) (width 0.2) (layer "F.Cu") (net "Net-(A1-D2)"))
 (segment (start 141.924998 107.545) (end 138.544998 107.545) (width 0.2) (layer "F.Cu") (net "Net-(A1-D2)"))
 (segment (start 138.544998 107.545) (end 132.089998 114) (width 0.2) (layer "F.Cu") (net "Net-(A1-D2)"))
 (segment (start 138.499998 105) (end 135.499998 108) (width 0.2) (layer "F.Cu") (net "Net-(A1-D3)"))
 (segment (start 135.499998 108) (end 128.999998 108) (width 0.2) (layer "F.Cu") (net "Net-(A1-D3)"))
 (segment (start 138.504998 105.005) (end 138.499998 105) (width 0.2) (layer "F.Cu") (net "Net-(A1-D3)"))
 (segment (start 141.924998 105.005) (end 138.504998 105.005) (width 0.2) (layer "F.Cu") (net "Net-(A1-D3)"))
 (segment (start 138.499998 102.5) (end 137.499998 101.5) (width 0.2) (layer "F.Cu") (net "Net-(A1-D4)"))
 (segment (start 137.499998 101.5) (end 128.999998 101.5) (width 0.2) (layer "F.Cu") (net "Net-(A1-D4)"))
 (segment (start 138.534998 102.465) (end 138.499998 102.5) (width 0.2) (layer "F.Cu") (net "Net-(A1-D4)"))
 (segment (start 141.924998 102.465) (end 138.534998 102.465) (width 0.2) (layer "F.Cu") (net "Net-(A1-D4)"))
 (segment (start 138.499998 99.925) (end 138.499998 95.5) (width 0.2) (layer "F.Cu") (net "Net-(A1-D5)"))
 (segment (start 134.999998 92) (end 128.999998 92) (width 0.2) (layer "F.Cu") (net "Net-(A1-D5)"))
 (segment (start 141.924998 99.925) (end 138.499998 99.925) (width 0.2) (layer "F.Cu") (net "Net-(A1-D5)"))
 (segment (start 138.499998 95.5) (end 134.999998 92) (width 0.2) (layer "F.Cu") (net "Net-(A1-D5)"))
 (segment (start 141.924998 97.385) (end 130.519998 85.98) (width 0.2) (layer "F.Cu") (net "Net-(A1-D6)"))
 (segment (start 130.519998 82.52) (end 130.499998 82.5) (width 0.2) (layer "F.Cu") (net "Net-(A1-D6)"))
 (segment (start 130.519998 85.98) (end 130.519998 82.52) (width 0.2) (layer "F.Cu") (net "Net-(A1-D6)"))
 (segment (start 130.499998 82.5) (end 128.999998 82.5) (width 0.2) (layer "F.Cu") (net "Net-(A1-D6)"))
 (segment (start 141.924998 94.845) (end 131.499998 84.42) (width 0.2) (layer "F.Cu") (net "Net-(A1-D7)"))
 (segment (start 131.499998 84.42) (end 131.499998 76) (width 0.2) (layer "F.Cu") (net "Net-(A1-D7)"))
 (segment (start 131.499998 76) (end 128.999998 76) (width 0.2) (layer "F.Cu") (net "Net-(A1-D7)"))
 (segment (start 118.839998 76) (end 107.499998 76) (width 0.2) (layer "F.Cu") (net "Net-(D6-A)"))
 (segment (start 107.499998 76) (end 106.839998 76.66) (width 0.2) (layer "F.Cu") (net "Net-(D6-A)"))
 (segment (start 106.839998 76.66) (end 106.839998 82.5) (width 0.2) (layer "F.Cu") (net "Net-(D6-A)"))
 (segment (start 118.839998 92) (end 106.879998 92) (width 0.2) (layer "F.Cu") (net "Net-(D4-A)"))
 (segment (start 99.839998 107.34) (end 99.839998 101.5) (width 0.2) (layer "F.Cu") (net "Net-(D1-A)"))
 (segment (start 112.499998 114) (end 105.999998 107.5) (width 0.2) (layer "F.Cu") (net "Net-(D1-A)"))
 (segment (start 99.999998 107.5) (end 99.839998 107.34) (width 0.2) (layer "F.Cu") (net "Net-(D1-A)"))
 (segment (start 118.839998 114) (end 112.499998 114) (width 0.2) (layer "F.Cu") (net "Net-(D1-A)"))
 (segment (start 105.999998 107.5) (end 99.999998 107.5) (width 0.2) (layer "F.Cu") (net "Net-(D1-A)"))
 (segment (start 214.159998 74) (end 220.659998 74) (width 0.2) (layer "F.Cu") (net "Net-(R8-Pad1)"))
 (segment (start 212.159998 76) (end 214.159998 74) (width 0.2) (layer "F.Cu") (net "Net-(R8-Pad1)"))
 (segment (start 209.659998 84.5) (end 212.159998 84.5) (width 0.2) (layer "F.Cu") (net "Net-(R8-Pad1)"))
 (segment (start 212.159998 84.5) (end 212.159998 76) (width 0.2) (layer "F.Cu") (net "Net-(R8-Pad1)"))
 (segment (start 118.839998 82.5) (end 113.839998 82.5) (width 0.2) (layer "F.Cu") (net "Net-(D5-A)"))
 (segment (start 107.499998 108) (end 106.839998 107.34) (width 0.2) (layer "F.Cu") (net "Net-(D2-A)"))
 (segment (start 118.839998 108) (end 107.499998 108) (width 0.2) (layer "F.Cu") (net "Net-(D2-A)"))
 (segment (start 106.839998 107.34) (end 106.839998 101.5) (width 0.2) (layer "F.Cu") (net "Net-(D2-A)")))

